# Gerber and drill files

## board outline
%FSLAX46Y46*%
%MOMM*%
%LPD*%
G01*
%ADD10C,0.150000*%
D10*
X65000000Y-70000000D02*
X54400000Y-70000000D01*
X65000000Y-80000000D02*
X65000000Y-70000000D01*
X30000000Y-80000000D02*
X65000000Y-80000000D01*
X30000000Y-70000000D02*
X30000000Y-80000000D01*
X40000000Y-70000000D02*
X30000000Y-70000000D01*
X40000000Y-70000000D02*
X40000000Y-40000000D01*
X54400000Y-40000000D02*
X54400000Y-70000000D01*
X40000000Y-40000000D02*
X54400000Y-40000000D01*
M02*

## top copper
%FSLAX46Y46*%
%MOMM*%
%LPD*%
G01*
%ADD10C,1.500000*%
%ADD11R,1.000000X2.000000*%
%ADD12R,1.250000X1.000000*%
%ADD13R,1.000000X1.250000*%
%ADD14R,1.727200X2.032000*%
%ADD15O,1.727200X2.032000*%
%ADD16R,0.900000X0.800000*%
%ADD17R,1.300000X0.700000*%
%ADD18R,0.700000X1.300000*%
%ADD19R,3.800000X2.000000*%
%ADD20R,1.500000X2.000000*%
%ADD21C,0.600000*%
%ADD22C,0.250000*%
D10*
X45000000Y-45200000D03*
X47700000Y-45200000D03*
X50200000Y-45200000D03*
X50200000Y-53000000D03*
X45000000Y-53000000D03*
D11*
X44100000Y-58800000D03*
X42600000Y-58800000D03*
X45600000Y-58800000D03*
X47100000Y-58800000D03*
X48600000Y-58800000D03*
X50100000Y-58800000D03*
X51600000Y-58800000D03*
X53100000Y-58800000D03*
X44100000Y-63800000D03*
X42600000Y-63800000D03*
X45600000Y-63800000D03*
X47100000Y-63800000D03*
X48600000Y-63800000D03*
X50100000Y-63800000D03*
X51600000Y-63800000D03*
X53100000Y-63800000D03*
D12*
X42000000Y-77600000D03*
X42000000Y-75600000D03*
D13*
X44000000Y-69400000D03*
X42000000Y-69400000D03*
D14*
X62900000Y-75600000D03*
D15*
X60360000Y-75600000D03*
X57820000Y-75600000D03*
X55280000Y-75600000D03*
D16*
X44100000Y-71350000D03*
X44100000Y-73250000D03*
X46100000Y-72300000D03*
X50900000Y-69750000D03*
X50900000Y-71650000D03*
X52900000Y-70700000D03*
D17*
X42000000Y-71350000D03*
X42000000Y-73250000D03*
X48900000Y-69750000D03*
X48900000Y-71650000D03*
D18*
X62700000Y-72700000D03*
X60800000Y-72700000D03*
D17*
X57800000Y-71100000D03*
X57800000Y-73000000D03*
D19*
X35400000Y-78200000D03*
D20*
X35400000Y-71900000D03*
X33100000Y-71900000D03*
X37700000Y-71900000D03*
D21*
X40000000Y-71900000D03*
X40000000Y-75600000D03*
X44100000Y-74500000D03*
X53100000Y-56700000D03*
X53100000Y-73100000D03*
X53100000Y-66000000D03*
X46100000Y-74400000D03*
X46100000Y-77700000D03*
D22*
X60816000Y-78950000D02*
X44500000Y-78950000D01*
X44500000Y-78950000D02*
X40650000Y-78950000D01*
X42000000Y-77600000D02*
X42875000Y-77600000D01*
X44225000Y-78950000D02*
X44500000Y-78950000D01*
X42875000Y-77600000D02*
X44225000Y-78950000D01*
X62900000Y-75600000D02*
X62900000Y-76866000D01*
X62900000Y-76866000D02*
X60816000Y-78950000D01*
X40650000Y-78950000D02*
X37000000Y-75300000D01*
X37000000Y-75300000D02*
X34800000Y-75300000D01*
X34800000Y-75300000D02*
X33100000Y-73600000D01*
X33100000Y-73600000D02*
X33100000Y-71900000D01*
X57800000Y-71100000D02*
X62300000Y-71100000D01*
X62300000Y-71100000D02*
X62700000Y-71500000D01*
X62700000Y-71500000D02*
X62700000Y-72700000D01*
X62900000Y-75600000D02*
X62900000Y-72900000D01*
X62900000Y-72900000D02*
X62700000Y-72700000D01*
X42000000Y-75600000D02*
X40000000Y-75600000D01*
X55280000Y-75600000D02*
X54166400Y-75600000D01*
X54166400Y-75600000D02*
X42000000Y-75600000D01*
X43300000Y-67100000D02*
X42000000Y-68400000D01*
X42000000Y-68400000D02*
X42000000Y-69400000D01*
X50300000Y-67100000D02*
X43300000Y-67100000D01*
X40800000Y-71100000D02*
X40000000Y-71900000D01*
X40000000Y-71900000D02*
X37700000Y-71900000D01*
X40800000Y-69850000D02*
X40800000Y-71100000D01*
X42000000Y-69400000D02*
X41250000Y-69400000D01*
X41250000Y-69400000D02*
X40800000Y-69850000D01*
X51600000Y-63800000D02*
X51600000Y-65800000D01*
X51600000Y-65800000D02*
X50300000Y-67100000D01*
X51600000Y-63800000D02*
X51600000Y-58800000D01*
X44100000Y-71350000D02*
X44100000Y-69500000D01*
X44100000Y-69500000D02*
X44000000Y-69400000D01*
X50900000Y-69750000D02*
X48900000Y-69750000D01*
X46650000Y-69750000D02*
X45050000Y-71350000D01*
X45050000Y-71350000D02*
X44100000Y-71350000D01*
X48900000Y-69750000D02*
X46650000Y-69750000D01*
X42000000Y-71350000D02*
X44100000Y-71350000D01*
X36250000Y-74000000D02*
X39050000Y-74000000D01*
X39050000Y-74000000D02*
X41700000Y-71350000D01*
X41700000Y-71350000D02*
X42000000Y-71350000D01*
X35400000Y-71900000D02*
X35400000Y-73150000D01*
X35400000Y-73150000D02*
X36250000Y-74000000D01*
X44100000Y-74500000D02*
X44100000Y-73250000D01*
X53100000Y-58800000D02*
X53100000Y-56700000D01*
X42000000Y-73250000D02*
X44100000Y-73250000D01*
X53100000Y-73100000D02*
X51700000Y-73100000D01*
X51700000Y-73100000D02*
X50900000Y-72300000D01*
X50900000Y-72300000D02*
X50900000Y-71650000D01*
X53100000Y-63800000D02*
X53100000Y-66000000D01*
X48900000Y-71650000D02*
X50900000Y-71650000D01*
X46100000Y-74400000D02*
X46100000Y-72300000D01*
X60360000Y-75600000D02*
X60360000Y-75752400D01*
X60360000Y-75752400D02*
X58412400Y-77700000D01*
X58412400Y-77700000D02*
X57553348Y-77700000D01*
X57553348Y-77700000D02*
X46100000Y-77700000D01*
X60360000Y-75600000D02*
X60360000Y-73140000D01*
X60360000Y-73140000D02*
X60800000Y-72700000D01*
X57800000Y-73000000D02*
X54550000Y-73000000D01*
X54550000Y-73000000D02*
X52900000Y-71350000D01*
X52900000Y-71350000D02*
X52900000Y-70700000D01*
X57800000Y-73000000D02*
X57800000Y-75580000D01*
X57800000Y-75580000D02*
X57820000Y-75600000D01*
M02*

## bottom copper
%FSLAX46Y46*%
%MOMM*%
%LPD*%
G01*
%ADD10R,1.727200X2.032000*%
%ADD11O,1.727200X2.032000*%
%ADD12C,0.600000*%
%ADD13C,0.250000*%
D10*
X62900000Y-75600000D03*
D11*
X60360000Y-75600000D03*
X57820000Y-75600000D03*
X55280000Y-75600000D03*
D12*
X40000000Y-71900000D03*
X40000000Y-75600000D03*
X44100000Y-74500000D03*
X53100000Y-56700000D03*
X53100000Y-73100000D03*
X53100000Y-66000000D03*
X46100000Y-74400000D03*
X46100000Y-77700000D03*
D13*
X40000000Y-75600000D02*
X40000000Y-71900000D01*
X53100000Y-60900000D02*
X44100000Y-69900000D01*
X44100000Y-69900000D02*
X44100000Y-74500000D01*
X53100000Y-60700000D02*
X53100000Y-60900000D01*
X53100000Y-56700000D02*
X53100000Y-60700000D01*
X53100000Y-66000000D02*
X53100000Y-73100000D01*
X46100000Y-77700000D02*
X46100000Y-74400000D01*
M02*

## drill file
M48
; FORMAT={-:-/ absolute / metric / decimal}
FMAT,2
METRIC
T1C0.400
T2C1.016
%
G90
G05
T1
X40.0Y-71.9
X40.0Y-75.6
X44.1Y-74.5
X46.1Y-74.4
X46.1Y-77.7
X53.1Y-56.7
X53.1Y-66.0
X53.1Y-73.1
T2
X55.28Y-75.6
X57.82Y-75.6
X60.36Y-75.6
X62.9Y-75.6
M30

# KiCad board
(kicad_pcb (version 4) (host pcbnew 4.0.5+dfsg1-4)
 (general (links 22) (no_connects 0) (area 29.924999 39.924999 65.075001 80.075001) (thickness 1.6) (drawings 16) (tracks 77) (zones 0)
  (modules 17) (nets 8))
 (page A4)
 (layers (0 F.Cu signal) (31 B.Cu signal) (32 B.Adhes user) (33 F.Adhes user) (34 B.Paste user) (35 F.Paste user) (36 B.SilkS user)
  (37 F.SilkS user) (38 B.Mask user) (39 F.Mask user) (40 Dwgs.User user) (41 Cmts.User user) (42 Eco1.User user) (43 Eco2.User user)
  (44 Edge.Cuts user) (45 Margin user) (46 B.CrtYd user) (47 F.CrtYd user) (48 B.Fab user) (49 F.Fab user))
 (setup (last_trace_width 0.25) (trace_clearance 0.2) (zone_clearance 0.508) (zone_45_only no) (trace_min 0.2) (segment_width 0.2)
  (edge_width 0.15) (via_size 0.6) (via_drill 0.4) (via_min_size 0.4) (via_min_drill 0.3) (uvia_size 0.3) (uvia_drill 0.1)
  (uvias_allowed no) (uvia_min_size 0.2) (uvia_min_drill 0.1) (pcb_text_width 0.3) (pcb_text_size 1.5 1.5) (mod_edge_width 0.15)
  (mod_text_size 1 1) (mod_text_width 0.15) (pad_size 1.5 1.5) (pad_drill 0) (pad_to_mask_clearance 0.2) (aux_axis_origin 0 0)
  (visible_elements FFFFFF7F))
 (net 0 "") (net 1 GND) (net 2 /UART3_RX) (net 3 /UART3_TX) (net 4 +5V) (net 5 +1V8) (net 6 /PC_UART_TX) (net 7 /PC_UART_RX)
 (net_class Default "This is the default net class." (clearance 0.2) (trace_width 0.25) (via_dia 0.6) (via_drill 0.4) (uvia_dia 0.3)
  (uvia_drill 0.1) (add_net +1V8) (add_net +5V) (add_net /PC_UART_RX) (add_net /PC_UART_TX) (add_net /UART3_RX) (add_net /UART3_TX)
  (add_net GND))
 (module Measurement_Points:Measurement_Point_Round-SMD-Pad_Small (layer F.Cu) (at 45 45.2)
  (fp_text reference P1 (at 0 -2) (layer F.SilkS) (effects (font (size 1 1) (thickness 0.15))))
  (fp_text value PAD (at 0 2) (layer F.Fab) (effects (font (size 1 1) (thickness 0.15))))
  (pad 1 smd circle (at 0 0) (size 1.5 1.5) (layers F.Cu F.Mask)))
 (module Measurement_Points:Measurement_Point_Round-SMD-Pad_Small (layer F.Cu) (at 47.7 45.2)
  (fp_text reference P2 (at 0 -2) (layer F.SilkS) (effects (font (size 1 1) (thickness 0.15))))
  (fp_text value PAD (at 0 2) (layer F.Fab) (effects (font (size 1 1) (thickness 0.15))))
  (pad 1 smd circle (at 0 0) (size 1.5 1.5) (layers F.Cu F.Mask)))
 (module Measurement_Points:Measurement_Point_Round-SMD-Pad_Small (layer F.Cu) (at 50.2 45.2)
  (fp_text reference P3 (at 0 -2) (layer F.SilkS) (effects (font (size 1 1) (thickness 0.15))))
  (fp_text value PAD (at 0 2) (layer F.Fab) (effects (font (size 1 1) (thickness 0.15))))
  (pad 1 smd circle (at 0 0) (size 1.5 1.5) (layers F.Cu F.Mask)))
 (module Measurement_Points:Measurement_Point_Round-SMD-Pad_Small (layer F.Cu) (at 50.2 53)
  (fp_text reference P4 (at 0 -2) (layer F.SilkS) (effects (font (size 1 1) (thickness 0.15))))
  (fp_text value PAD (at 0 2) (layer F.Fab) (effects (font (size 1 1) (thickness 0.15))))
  (pad 1 smd circle (at 0 0) (size 1.5 1.5) (layers F.Cu F.Mask)))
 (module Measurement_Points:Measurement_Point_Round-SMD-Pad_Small (layer F.Cu) (at 45 53)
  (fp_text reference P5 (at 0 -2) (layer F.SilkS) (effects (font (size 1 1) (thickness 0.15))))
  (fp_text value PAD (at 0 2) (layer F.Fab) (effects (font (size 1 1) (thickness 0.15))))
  (pad 1 smd circle (at 0 0) (size 1.5 1.5) (layers F.Cu F.Mask)))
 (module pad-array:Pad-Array (layer F.Cu) (at 47.85 58.8)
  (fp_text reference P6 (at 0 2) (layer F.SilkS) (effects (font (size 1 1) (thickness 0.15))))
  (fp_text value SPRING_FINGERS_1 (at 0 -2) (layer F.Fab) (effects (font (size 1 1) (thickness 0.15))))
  (pad 2 smd rect (at -3.75 0) (size 1 2) (layers F.Cu F.Paste F.Mask))
  (pad 1 smd rect (at -5.25 0) (size 1 2) (layers F.Cu F.Paste F.Mask))
  (pad 3 smd rect (at -2.25 0) (size 1 2) (layers F.Cu F.Paste F.Mask))
  (pad 4 smd rect (at -0.75 0) (size 1 2) (layers F.Cu F.Paste F.Mask))
  (pad 5 smd rect (at 0.75 0) (size 1 2) (layers F.Cu F.Paste F.Mask))
  (pad 6 smd rect (at 2.25 0) (size 1 2) (layers F.Cu F.Paste F.Mask))
  (pad 7 smd rect (at 3.75 0) (size 1 2) (layers F.Cu F.Paste F.Mask) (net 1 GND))
  (pad 8 smd rect (at 5.25 0) (size 1 2) (layers F.Cu F.Paste F.Mask) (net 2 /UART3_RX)))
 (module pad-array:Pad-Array (layer F.Cu) (at 47.85 63.8)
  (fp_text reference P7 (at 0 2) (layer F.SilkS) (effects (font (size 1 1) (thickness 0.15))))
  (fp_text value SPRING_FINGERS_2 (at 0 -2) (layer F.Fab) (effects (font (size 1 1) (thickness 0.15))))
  (pad 2 smd rect (at -3.75 0) (size 1 2) (layers F.Cu F.Paste F.Mask))
  (pad 1 smd rect (at -5.25 0) (size 1 2) (layers F.Cu F.Paste F.Mask))
  (pad 3 smd rect (at -2.25 0) (size 1 2) (layers F.Cu F.Paste F.Mask))
  (pad 4 smd rect (at -0.75 0) (size 1 2) (layers F.Cu F.Paste F.Mask))
  (pad 5 smd rect (at 0.75 0) (size 1 2) (layers F.Cu F.Paste F.Mask))
  (pad 6 smd rect (at 2.25 0) (size 1 2) (layers F.Cu F.Paste F.Mask))
  (pad 7 smd rect (at 3.75 0) (size 1 2) (layers F.Cu F.Paste F.Mask) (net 1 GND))
  (pad 8 smd rect (at 5.25 0) (size 1 2) (layers F.Cu F.Paste F.Mask) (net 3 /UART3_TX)))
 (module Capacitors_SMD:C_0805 (layer F.Cu) (at 42 76.6 90)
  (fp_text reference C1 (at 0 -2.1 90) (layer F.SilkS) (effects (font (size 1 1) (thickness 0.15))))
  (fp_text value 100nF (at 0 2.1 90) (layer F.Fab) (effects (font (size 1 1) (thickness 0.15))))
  (pad 1 smd rect (at -1 0 90) (size 1 1.25) (layers F.Cu F.Paste F.Mask) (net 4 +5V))
  (pad 2 smd rect (at 1 0 90) (size 1 1.25) (layers F.Cu F.Paste F.Mask) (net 1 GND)))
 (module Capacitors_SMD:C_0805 (layer F.Cu) (at 43 69.4 180)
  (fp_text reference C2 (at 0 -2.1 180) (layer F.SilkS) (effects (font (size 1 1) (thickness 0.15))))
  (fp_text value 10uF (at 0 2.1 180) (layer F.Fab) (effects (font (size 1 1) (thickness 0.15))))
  (pad 1 smd rect (at -1 0 180) (size 1 1.25) (layers F.Cu F.Paste F.Mask) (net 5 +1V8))
  (pad 2 smd rect (at 1 0 180) (size 1 1.25) (layers F.Cu F.Paste F.Mask) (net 1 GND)))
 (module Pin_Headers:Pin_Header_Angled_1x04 (layer F.Cu) (at 62.9 75.6 270)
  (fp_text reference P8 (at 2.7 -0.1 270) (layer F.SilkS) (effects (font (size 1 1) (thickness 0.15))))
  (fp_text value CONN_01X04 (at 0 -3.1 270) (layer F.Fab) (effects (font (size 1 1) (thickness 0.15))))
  (pad 1 thru_hole rect (at 0 0 270) (size 2.032 1.7272) (drill 1.016) (layers *.Cu *.Mask) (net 4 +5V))
  (pad 2 thru_hole oval (at 0 2.54 270) (size 2.032 1.7272) (drill 1.016) (layers *.Cu *.Mask) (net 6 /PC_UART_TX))
  (pad 3 thru_hole oval (at 0 5.08 270) (size 2.032 1.7272) (drill 1.016) (layers *.Cu *.Mask) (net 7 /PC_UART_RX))
  (pad 4 thru_hole oval (at 0 7.62 270) (size 2.032 1.7272) (drill 1.016) (layers *.Cu *.Mask) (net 1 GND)))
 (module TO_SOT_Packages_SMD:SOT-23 (layer F.Cu) (at 45.1 72.3)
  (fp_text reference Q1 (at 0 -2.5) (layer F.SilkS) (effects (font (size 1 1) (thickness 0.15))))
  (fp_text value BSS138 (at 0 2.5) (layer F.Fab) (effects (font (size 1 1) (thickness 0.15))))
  (pad 1 smd rect (at -1 -0.95) (size 0.9 0.8) (layers F.Cu F.Paste F.Mask) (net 5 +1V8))
  (pad 2 smd rect (at -1 0.95) (size 0.9 0.8) (layers F.Cu F.Paste F.Mask) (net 2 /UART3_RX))
  (pad 3 smd rect (at 1 0) (size 0.9 0.8) (layers F.Cu F.Paste F.Mask) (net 6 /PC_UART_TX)))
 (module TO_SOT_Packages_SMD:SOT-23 (layer F.Cu) (at 51.9 70.7)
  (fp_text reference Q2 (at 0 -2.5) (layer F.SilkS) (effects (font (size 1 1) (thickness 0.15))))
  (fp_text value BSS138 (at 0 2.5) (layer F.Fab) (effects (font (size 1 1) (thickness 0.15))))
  (pad 1 smd rect (at -1 -0.95) (size 0.9 0.8) (layers F.Cu F.Paste F.Mask) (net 5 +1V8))
  (pad 2 smd rect (at -1 0.95) (size 0.9 0.8) (layers F.Cu F.Paste F.Mask) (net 3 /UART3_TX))
  (pad 3 smd rect (at 1 0) (size 0.9 0.8) (layers F.Cu F.Paste F.Mask) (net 7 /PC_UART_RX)))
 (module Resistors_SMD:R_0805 (layer F.Cu) (at 42 72.3 270)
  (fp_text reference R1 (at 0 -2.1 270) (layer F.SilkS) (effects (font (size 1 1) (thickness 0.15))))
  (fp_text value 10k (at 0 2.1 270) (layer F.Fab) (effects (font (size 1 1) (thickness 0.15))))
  (pad 1 smd rect (at -0.95 0 270) (size 0.7 1.3) (layers F.Cu F.Paste F.Mask) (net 5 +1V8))
  (pad 2 smd rect (at 0.95 0 270) (size 0.7 1.3) (layers F.Cu F.Paste F.Mask) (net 2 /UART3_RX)))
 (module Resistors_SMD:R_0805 (layer F.Cu) (at 48.9 70.7 270)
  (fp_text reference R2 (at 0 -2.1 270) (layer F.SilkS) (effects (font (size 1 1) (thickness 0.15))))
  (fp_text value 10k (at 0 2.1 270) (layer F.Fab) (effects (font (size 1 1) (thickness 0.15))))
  (pad 1 smd rect (at -0.95 0 270) (size 0.7 1.3) (layers F.Cu F.Paste F.Mask) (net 5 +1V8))
  (pad 2 smd rect (at 0.95 0 270) (size 0.7 1.3) (layers F.Cu F.Paste F.Mask) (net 3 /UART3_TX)))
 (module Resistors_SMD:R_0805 (layer F.Cu) (at 61.75 72.7 180)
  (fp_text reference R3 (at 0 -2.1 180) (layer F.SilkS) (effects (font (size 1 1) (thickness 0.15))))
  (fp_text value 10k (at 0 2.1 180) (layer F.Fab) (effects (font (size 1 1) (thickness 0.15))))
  (pad 1 smd rect (at -0.95 0 180) (size 0.7 1.3) (layers F.Cu F.Paste F.Mask) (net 4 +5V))
  (pad 2 smd rect (at 0.95 0 180) (size 0.7 1.3) (layers F.Cu F.Paste F.Mask) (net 6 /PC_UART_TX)))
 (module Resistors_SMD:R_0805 (layer F.Cu) (at 57.8 72.05 270)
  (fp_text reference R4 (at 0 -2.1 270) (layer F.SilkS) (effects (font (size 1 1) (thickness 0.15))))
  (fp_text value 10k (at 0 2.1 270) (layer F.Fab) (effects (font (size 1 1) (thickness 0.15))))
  (pad 1 smd rect (at -0.95 0 270) (size 0.7 1.3) (layers F.Cu F.Paste F.Mask) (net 4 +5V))
  (pad 2 smd rect (at 0.95 0 270) (size 0.7 1.3) (layers F.Cu F.Paste F.Mask) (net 7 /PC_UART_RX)))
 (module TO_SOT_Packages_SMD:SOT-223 (layer F.Cu) (at 35.4 75.05 270)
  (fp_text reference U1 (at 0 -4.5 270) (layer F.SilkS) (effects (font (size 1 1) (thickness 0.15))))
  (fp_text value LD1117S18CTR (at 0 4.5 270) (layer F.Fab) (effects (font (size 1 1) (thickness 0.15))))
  (pad 4 smd rect (at 3.15 0 270) (size 2 3.8) (layers F.Cu F.Paste F.Mask))
  (pad 2 smd rect (at -3.15 0 270) (size 2 1.5) (layers F.Cu F.Paste F.Mask) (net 5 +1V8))
  (pad 3 smd rect (at -3.15 2.3 270) (size 2 1.5) (layers F.Cu F.Paste F.Mask) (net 4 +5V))
  (pad 1 smd rect (at -3.15 -2.3 270) (size 2 1.5) (layers F.Cu F.Paste F.Mask) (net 1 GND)))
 (gr_line (start 65 70) (end 54.4 70) (layer Edge.Cuts) (width 0.15))
 (gr_line (start 65 80) (end 65 70) (layer Edge.Cuts) (width 0.15))
 (gr_line (start 30 80) (end 65 80) (layer Edge.Cuts) (width 0.15))
 (gr_line (start 30 70) (end 30 80) (layer Edge.Cuts) (width 0.15))
 (gr_line (start 40 70) (end 30 70) (layer Edge.Cuts) (width 0.15))
 (gr_line (start 40 70) (end 40 40) (layer Edge.Cuts) (width 0.15))
 (gr_line (start 54.4 40) (end 54.4 70) (layer Edge.Cuts) (width 0.15))
 (gr_line (start 40 40) (end 54.4 40) (layer Edge.Cuts) (width 0.15))
 (segment (start 60.816 78.95) (end 44.5 78.95) (width 0.25) (layer F.Cu) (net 4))
 (segment (start 44.5 78.95) (end 40.65 78.95) (width 0.25) (layer F.Cu) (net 4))
 (segment (start 42 77.6) (end 42.875 77.6) (width 0.25) (layer F.Cu) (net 4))
 (segment (start 44.225 78.95) (end 44.5 78.95) (width 0.25) (layer F.Cu) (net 4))
 (segment (start 42.875 77.6) (end 44.225 78.95) (width 0.25) (layer F.Cu) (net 4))
 (segment (start 62.9 75.6) (end 62.9 76.866) (width 0.25) (layer F.Cu) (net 4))
 (segment (start 62.9 76.866) (end 60.816 78.95) (width 0.25) (layer F.Cu) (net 4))
 (segment (start 40.65 78.95) (end 37 75.3) (width 0.25) (layer F.Cu) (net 4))
 (segment (start 37 75.3) (end 34.8 75.3) (width 0.25) (layer F.Cu) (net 4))
 (segment (start 34.8 75.3) (end 33.1 73.6) (width 0.25) (layer F.Cu) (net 4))
 (segment (start 33.1 73.6) (end 33.1 71.9) (width 0.25) (layer F.Cu) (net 4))
 (segment (start 57.8 71.1) (end 62.3 71.1) (width 0.25) (layer F.Cu) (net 4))
 (segment (start 62.3 71.1) (end 62.7 71.5) (width 0.25) (layer F.Cu) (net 4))
 (segment (start 62.7 71.5) (end 62.7 72.7) (width 0.25) (layer F.Cu) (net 4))
 (segment (start 62.9 75.6) (end 62.9 72.9) (width 0.25) (layer F.Cu) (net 4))
 (segment (start 62.9 72.9) (end 62.7 72.7) (width 0.25) (layer F.Cu) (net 4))
 (segment (start 40 75.6) (end 40 71.9) (width 0.25) (layer B.Cu) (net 1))
 (via (at 40 71.9) (size 0.6) (drill 0.4) (layers F.Cu B.Cu) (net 1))
 (segment (start 42 75.6) (end 40 75.6) (width 0.25) (layer F.Cu) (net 1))
 (via (at 40 75.6) (size 0.6) (drill 0.4) (layers F.Cu B.Cu) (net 1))
 (segment (start 55.28 75.6) (end 54.1664 75.6) (width 0.25) (layer F.Cu) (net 1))
 (segment (start 54.1664 75.6) (end 42 75.6) (width 0.25) (layer F.Cu) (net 1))
 (segment (start 43.3 67.1) (end 42 68.4) (width 0.25) (layer F.Cu) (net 1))
 (segment (start 42 68.4) (end 42 69.4) (width 0.25) (layer F.Cu) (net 1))
 (segment (start 50.3 67.1) (end 43.3 67.1) (width 0.25) (layer F.Cu) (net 1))
 (segment (start 40.8 71.1) (end 40 71.9) (width 0.25) (layer F.Cu) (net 1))
 (segment (start 40 71.9) (end 37.7 71.9) (width 0.25) (layer F.Cu) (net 1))
 (segment (start 40.8 69.85) (end 40.8 71.1) (width 0.25) (layer F.Cu) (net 1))
 (segment (start 42 69.4) (end 41.25 69.4) (width 0.25) (layer F.Cu) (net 1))
 (segment (start 41.25 69.4) (end 40.8 69.85) (width 0.25) (layer F.Cu) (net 1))
 (segment (start 51.6 63.8) (end 51.6 65.8) (width 0.25) (layer F.Cu) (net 1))
 (segment (start 51.6 65.8) (end 50.3 67.1) (width 0.25) (layer F.Cu) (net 1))
 (segment (start 51.6 63.8) (end 51.6 58.8) (width 0.25) (layer F.Cu) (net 1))
 (segment (start 44.1 71.35) (end 44.1 69.5) (width 0.25) (layer F.Cu) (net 5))
 (segment (start 44.1 69.5) (end 44 69.4) (width 0.25) (layer F.Cu) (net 5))
 (segment (start 50.9 69.75) (end 48.9 69.75) (width 0.25) (layer F.Cu) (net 5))
 (segment (start 46.65 69.75) (end 45.05 71.35) (width 0.25) (layer F.Cu) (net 5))
 (segment (start 45.05 71.35) (end 44.1 71.35) (width 0.25) (layer F.Cu) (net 5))
 (segment (start 48.9 69.75) (end 46.65 69.75) (width 0.25) (layer F.Cu) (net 5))
 (segment (start 42 71.35) (end 44.1 71.35) (width 0.25) (layer F.Cu) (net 5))
 (segment (start 36.25 74) (end 39.05 74) (width 0.25) (layer F.Cu) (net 5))
 (segment (start 39.05 74) (end 41.7 71.35) (width 0.25) (layer F.Cu) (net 5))
 (segment (start 41.7 71.35) (end 42 71.35) (width 0.25) (layer F.Cu) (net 5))
 (segment (start 35.4 71.9) (end 35.4 73.15) (width 0.25) (layer F.Cu) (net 5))
 (segment (start 35.4 73.15) (end 36.25 74) (width 0.25) (layer F.Cu) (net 5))
 (segment (start 44.1 74.5) (end 44.1 73.25) (width 0.25) (layer F.Cu) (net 2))
 (segment (start 53.1 60.9) (end 44.1 69.9) (width 0.25) (layer B.Cu) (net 2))
 (segment (start 44.1 69.9) (end 44.1 74.5) (width 0.25) (layer B.Cu) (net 2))
 (via (at 44.1 74.5) (size 0.6) (drill 0.4) (layers F.Cu B.Cu) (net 2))
 (segment (start 53.1 60.7) (end 53.1 60.9) (width 0.25) (layer B.Cu) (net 2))
 (segment (start 53.1 56.7) (end 53.1 60.7) (width 0.25) (layer B.Cu) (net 2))
 (segment (start 53.1 58.8) (end 53.1 56.7) (width 0.25) (layer F.Cu) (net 2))
 (via (at 53.1 56.7) (size 0.6) (drill 0.4) (layers F.Cu B.Cu) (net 2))
 (segment (start 42 73.25) (end 44.1 73.25) (width 0.25) (layer F.Cu) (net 2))
 (segment (start 53.1 73.1) (end 51.7 73.1) (width 0.25) (layer F.Cu) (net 3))
 (segment (start 51.7 73.1) (end 50.9 72.3) (width 0.25) (layer F.Cu) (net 3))
 (segment (start 50.9 72.3) (end 50.9 71.65) (width 0.25) (layer F.Cu) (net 3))
 (segment (start 53.1 66) (end 53.1 73.1) (width 0.25) (layer B.Cu) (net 3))
 (via (at 53.1 73.1) (size 0.6) (drill 0.4) (layers F.Cu B.Cu) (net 3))
 (segment (start 53.1 63.8) (end 53.1 66) (width 0.25) (layer F.Cu) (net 3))
 (via (at 53.1 66) (size 0.6) (drill 0.4) (layers F.Cu B.Cu) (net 3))
 (segment (start 48.9 71.65) (end 50.9 71.65) (width 0.25) (layer F.Cu) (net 3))
 (segment (start 46.1 74.4) (end 46.1 72.3) (width 0.25) (layer F.Cu) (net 6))
 (segment (start 46.1 77.7) (end 46.1 74.4) (width 0.25) (layer B.Cu) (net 6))
 (via (at 46.1 74.4) (size 0.6) (drill 0.4) (layers F.Cu B.Cu) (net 6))
 (segment (start 60.36 75.6) (end 60.36 75.7524) (width 0.25) (layer F.Cu) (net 6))
 (segment (start 60.36 75.7524) (end 58.4124 77.7) (width 0.25) (layer F.Cu) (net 6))
 (segment (start 58.4124 77.7) (end 57.553348 77.7) (width 0.25) (layer F.Cu) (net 6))
 (segment (start 57.553348 77.7) (end 46.1 77.7) (width 0.25) (layer F.Cu) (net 6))
 (via (at 46.1 77.7) (size 0.6) (drill 0.4) (layers F.Cu B.Cu) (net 6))
 (segment (start 60.36 75.6) (end 60.36 73.14) (width 0.25) (layer F.Cu) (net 6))
 (segment (start 60.36 73.14) (end 60.8 72.7) (width 0.25) (layer F.Cu) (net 6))
 (segment (start 57.8 73) (end 54.55 73) (width 0.25) (layer F.Cu) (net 7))
 (segment (start 54.55 73) (end 52.9 71.35) (width 0.25) (layer F.Cu) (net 7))
 (segment (start 52.9 71.35) (end 52.9 70.7) (width 0.25) (layer F.Cu) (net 7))
 (segment (start 57.8 73) (end 57.8 75.58) (width 0.25) (layer F.Cu) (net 7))
 (segment (start 57.8 75.58) (end 57.82 75.6) (width 0.25) (layer F.Cu) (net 7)))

